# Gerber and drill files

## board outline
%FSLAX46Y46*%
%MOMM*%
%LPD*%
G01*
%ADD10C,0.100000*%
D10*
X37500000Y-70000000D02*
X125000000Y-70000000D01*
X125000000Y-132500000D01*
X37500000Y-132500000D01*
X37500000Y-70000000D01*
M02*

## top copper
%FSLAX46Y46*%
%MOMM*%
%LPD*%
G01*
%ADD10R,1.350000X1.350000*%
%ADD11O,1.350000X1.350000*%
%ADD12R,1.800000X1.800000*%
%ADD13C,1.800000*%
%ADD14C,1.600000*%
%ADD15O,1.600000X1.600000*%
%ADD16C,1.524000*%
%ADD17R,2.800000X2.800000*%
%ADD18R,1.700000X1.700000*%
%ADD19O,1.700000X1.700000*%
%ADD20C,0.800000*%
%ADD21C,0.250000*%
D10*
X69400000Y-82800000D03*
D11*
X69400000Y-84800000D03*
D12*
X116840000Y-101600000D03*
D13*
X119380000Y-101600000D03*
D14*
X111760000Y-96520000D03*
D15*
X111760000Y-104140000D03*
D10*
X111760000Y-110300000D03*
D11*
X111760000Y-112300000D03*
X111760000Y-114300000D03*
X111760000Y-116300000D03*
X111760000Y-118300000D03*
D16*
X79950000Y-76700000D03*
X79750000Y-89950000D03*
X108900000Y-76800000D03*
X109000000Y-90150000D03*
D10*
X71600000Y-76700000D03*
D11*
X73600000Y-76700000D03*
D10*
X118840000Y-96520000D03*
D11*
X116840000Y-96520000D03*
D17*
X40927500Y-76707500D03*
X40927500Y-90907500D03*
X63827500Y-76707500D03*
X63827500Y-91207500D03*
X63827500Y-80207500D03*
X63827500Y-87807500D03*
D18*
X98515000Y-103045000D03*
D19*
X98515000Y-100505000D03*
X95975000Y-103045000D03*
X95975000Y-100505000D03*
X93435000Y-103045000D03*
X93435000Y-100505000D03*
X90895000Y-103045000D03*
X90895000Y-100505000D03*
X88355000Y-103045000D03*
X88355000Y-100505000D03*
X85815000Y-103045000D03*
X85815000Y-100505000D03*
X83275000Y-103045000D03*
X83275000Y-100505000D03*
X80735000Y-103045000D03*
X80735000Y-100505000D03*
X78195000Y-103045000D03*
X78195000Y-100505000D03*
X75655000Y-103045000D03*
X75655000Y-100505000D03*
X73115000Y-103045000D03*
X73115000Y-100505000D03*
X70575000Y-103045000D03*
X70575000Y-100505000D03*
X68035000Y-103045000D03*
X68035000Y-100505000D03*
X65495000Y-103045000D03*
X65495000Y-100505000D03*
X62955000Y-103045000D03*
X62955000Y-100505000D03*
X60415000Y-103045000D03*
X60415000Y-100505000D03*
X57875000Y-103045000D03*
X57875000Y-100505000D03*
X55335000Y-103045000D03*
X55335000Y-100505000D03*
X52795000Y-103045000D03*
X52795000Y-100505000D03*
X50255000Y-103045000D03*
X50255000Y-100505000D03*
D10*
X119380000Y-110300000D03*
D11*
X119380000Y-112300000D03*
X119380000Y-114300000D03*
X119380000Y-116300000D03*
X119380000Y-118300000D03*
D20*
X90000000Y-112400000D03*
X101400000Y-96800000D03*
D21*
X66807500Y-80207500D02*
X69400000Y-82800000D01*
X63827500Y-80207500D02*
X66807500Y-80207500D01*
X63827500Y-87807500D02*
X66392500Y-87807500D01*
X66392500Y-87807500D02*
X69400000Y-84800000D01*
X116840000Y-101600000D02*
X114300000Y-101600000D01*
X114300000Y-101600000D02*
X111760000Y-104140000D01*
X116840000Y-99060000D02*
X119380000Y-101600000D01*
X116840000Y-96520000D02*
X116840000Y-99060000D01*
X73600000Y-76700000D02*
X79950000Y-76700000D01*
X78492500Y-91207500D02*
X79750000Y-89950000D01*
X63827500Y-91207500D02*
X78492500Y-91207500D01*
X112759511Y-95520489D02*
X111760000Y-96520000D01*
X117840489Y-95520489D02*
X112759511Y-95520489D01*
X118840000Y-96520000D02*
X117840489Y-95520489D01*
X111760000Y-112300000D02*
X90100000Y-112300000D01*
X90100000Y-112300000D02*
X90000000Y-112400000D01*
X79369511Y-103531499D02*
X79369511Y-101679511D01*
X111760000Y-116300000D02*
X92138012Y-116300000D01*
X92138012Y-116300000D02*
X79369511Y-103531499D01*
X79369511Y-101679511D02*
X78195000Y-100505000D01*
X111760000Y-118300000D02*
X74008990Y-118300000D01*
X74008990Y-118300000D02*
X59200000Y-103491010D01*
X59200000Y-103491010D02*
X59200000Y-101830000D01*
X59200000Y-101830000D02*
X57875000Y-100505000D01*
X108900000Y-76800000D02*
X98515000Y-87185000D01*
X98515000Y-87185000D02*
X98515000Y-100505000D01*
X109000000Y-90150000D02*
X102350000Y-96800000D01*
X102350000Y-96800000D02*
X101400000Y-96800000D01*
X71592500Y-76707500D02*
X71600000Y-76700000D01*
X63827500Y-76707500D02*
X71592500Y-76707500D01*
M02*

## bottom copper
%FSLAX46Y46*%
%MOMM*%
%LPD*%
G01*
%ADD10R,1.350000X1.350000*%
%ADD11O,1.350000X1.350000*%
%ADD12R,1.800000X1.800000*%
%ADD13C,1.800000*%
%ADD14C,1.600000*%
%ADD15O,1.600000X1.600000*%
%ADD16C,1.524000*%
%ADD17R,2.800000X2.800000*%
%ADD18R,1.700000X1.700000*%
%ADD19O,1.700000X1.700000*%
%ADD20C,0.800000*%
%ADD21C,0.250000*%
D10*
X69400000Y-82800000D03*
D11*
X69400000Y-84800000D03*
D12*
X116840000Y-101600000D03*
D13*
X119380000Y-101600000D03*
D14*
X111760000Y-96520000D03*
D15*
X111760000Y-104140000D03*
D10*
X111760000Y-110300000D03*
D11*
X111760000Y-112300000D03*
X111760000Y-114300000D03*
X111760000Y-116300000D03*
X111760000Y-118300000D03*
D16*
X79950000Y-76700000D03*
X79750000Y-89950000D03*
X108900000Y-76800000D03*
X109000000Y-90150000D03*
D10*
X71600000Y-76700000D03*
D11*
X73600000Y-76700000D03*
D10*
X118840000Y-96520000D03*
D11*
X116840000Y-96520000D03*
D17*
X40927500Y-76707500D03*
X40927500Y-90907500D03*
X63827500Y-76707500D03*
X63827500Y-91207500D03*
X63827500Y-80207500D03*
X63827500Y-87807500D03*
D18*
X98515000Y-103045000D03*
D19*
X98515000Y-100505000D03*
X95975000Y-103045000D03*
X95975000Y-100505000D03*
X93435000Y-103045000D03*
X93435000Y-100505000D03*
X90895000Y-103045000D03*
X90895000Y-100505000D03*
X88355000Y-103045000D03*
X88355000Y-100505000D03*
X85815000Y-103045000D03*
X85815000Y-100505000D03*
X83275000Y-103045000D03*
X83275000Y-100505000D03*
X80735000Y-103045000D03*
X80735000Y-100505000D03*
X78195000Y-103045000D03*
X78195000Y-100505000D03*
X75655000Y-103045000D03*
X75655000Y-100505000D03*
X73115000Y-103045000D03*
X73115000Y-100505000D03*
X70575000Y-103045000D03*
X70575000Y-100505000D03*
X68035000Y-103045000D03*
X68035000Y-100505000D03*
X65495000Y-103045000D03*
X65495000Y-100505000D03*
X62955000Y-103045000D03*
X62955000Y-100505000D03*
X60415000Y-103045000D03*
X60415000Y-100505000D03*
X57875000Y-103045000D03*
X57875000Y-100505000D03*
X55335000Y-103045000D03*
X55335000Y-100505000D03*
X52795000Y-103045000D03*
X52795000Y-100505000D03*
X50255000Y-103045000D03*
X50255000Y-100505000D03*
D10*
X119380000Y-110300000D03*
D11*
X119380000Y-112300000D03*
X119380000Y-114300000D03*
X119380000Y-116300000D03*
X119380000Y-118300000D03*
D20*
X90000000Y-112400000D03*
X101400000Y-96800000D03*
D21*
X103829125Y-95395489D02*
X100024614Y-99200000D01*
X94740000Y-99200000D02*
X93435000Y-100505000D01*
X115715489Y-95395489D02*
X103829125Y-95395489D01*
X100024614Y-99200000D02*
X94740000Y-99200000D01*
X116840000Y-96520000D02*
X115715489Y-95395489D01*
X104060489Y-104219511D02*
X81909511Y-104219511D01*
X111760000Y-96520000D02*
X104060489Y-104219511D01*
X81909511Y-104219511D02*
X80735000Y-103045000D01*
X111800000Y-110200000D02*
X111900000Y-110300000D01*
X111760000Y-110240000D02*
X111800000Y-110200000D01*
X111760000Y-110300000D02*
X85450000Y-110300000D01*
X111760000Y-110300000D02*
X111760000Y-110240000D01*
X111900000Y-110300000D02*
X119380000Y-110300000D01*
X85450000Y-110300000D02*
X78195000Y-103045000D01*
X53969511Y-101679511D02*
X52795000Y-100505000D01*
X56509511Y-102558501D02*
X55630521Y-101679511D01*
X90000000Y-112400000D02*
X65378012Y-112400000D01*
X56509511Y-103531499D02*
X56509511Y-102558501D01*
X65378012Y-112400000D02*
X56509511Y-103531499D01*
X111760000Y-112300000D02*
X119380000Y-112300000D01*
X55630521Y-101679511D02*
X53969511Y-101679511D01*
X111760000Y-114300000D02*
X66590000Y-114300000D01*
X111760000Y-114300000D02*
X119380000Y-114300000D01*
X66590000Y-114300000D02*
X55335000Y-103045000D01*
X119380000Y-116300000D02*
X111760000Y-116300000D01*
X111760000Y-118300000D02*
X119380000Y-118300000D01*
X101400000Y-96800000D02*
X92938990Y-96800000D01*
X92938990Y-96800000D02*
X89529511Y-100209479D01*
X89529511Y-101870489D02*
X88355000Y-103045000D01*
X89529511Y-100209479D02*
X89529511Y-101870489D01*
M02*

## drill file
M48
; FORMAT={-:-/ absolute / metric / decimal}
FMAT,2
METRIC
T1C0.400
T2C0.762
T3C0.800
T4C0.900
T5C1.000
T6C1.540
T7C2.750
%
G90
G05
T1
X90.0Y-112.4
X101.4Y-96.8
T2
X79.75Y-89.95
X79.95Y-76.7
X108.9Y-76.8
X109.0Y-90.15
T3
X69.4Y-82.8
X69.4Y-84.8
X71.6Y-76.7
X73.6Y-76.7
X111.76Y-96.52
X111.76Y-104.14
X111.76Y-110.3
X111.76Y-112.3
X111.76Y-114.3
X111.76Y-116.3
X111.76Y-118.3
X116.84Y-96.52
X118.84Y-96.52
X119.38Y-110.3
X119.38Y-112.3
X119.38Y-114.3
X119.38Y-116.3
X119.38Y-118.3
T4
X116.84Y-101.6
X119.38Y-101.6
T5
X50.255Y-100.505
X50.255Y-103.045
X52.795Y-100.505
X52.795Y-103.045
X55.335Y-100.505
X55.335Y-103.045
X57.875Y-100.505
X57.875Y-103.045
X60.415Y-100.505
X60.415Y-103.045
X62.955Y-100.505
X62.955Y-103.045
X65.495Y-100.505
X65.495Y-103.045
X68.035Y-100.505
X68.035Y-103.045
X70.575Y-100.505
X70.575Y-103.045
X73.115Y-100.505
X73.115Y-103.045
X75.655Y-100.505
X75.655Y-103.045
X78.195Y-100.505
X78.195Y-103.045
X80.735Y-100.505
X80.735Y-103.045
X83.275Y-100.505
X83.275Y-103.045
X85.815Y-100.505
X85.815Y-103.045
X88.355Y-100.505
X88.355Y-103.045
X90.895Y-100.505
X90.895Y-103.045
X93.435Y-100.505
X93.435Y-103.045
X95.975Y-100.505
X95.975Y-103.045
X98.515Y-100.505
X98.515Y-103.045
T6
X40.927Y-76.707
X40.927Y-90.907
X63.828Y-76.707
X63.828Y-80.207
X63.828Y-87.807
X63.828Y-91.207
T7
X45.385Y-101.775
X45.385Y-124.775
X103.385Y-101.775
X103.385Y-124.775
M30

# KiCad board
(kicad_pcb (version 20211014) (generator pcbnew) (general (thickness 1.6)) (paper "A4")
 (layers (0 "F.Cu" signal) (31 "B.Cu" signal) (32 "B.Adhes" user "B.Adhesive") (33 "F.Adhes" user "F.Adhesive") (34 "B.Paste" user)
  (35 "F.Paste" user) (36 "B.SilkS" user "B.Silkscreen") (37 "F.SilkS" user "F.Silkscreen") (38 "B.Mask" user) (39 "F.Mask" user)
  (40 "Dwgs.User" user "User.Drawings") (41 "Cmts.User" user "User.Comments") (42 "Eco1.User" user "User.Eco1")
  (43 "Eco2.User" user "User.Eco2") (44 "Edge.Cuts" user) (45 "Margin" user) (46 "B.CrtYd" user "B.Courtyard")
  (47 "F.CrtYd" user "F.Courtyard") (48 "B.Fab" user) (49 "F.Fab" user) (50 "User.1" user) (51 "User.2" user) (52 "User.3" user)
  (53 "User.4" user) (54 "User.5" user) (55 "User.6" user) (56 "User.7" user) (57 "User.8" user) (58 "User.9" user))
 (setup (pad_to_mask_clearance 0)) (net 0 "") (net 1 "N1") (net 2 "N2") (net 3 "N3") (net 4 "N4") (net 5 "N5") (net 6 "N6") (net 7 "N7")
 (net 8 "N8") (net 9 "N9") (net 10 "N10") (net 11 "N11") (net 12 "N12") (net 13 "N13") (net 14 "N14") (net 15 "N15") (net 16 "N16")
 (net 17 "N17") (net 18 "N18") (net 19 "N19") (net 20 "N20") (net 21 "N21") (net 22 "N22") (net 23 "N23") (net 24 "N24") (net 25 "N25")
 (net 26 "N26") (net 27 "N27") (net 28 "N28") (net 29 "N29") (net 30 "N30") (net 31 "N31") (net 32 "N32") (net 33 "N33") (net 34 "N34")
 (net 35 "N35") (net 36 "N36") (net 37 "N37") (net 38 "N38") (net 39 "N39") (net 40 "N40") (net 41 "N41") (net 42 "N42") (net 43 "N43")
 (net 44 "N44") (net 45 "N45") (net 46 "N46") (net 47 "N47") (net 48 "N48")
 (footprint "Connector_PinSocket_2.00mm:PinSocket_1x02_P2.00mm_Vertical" (layer "F.Cu") (at 69.4 82.8)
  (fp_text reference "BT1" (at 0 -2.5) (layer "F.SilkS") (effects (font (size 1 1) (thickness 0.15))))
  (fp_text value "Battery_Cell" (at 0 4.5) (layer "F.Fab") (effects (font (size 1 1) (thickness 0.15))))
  (pad "1" thru_hole rect (at 0 0) (size 1.35 1.35) (drill 0.8) (layers *.Cu *.Mask) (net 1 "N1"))
  (pad "2" thru_hole oval (at 0 2) (size 1.35 1.35) (drill 0.8) (layers *.Cu *.Mask) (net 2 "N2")))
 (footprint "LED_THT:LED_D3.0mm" (layer "F.Cu") (at 116.84 101.6)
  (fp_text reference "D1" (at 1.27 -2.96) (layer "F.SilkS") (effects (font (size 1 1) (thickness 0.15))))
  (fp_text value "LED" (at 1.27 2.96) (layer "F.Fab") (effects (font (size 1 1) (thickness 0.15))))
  (pad "1" thru_hole rect (at 0 0) (size 1.8 1.8) (drill 0.9) (layers *.Cu *.Mask) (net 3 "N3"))
  (pad "2" thru_hole circle (at 2.54 0) (size 1.8 1.8) (drill 0.9) (layers *.Cu *.Mask) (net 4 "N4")))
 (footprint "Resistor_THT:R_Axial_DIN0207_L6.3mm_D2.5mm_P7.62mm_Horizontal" (layer "F.Cu") (at 111.76 96.52 -90)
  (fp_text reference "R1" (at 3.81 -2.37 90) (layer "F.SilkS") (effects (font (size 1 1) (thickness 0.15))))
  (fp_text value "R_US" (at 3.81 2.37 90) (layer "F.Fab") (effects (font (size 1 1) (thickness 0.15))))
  (pad "1" thru_hole circle (at 0 0 270) (size 1.6 1.6) (drill 0.8) (layers *.Cu *.Mask) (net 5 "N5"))
  (pad "2" thru_hole oval (at 7.62 0 270) (size 1.6 1.6) (drill 0.8) (layers *.Cu *.Mask) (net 3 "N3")))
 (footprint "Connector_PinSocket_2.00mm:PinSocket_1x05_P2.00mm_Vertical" (layer "F.Cu") (at 111.76 110.3)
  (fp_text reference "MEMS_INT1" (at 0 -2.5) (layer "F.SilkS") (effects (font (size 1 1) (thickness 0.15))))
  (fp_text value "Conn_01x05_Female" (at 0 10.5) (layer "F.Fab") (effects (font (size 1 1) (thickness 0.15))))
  (pad "1" thru_hole rect (at 0 0) (size 1.35 1.35) (drill 0.8) (layers *.Cu *.Mask) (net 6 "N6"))
  (pad "2" thru_hole oval (at 0 2) (size 1.35 1.35) (drill 0.8) (layers *.Cu *.Mask) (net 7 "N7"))
  (pad "3" thru_hole oval (at 0 4) (size 1.35 1.35) (drill 0.8) (layers *.Cu *.Mask) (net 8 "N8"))
  (pad "4" thru_hole oval (at 0 6) (size 1.35 1.35) (drill 0.8) (layers *.Cu *.Mask) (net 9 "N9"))
  (pad "5" thru_hole oval (at 0 8) (size 1.35 1.35) (drill 0.8) (layers *.Cu *.Mask) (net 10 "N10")))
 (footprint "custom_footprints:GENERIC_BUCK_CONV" (layer "F.Cu") (at 94.2 83.6)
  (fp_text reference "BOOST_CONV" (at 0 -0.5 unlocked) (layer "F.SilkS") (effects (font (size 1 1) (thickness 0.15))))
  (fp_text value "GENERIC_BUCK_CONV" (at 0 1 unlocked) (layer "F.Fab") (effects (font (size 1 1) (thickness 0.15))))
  (pad "1" thru_hole circle (at -14.25 -6.9) (size 1.524 1.524) (drill 0.762) (layers *.Cu *.Mask) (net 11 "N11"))
  (pad "2" thru_hole circle (at -14.45 6.35) (size 1.524 1.524) (drill 0.762) (layers *.Cu *.Mask) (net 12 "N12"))
  (pad "3" thru_hole circle (at 14.7 -6.8) (size 1.524 1.524) (drill 0.762) (layers *.Cu *.Mask) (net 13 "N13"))
  (pad "4" thru_hole circle (at 14.8 6.55) (size 1.524 1.524) (drill 0.762) (layers *.Cu *.Mask) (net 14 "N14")))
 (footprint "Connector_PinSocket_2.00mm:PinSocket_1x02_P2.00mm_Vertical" (layer "F.Cu") (at 71.6 76.7 90)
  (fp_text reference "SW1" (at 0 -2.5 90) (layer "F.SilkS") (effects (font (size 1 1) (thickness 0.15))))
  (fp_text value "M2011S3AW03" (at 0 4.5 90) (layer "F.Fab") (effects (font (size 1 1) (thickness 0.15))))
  (pad "1" thru_hole rect (at 0 0 90) (size 1.35 1.35) (drill 0.8) (layers *.Cu *.Mask) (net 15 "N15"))
  (pad "2" thru_hole oval (at 0 2 90) (size 1.35 1.35) (drill 0.8) (layers *.Cu *.Mask) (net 11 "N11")))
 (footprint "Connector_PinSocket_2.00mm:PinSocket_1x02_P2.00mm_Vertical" (layer "F.Cu") (at 118.84 96.52 -90)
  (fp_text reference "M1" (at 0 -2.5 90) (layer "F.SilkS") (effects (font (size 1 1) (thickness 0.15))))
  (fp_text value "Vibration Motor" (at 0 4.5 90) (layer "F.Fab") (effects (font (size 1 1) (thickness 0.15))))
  (pad "1" thru_hole rect (at 0 0 270) (size 1.35 1.35) (drill 0.8) (layers *.Cu *.Mask) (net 5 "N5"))
  (pad "2" thru_hole oval (at 0 2 270) (size 1.35 1.35) (drill 0.8) (layers *.Cu *.Mask) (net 4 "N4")))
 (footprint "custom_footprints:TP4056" (layer "F.Cu") (at 39.2275 75.0075)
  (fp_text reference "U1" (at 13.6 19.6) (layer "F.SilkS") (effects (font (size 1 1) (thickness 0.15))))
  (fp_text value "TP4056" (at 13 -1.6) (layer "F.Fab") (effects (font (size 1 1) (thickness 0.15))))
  (pad "1" thru_hole rect (at 1.7 1.7) (size 2.8 2.8) (drill 1.54) (layers *.Cu *.Mask) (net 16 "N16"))
  (pad "2" thru_hole rect (at 1.7 15.9) (size 2.8 2.8) (drill 1.54) (layers *.Cu *.Mask) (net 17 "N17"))
  (pad "3" thru_hole rect (at 24.6 1.7) (size 2.8 2.8) (drill 1.54) (layers *.Cu *.Mask) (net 15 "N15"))
  (pad "4" thru_hole rect (at 24.6 16.2) (size 2.8 2.8) (drill 1.54) (layers *.Cu *.Mask) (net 12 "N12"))
  (pad "5" thru_hole rect (at 24.6 5.2) (size 2.8 2.8) (drill 1.54) (layers *.Cu *.Mask) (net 1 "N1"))
  (pad "6" thru_hole rect (at 24.6 12.8) (size 2.8 2.8) (drill 1.54) (layers *.Cu *.Mask) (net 2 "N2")))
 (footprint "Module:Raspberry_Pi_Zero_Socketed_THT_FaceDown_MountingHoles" (layer "F.Cu") (at 98.515 103.045 -90)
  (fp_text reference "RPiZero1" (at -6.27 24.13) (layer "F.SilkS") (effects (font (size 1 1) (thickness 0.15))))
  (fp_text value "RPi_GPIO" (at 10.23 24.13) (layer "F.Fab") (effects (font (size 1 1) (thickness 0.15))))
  (pad "" np_thru_hole circle (at 21.73 -4.87) (size 2.75 2.75) (drill 2.75) (layers *.Cu *.Mask) (solder_mask_margin 1.625))
  (pad "" np_thru_hole circle (at -1.27 53.13) (size 2.75 2.75) (drill 2.75) (layers *.Cu *.Mask) (solder_mask_margin 1.625))
  (pad "" np_thru_hole circle (at -1.27 -4.87) (size 2.75 2.75) (drill 2.75) (layers *.Cu *.Mask) (solder_mask_margin 1.625))
  (pad "" np_thru_hole circle (at 21.73 53.13) (size 2.75 2.75) (drill 2.75) (layers *.Cu *.Mask) (solder_mask_margin 1.625))
  (pad "1" thru_hole rect (at 0 0 270) (size 1.7 1.7) (drill 1) (layers *.Cu *.Mask) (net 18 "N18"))
  (pad "2" thru_hole oval (at -2.54 0 270) (size 1.7 1.7) (drill 1) (layers *.Cu *.Mask) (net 13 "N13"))
  (pad "3" thru_hole oval (at 0 2.54 270) (size 1.7 1.7) (drill 1) (layers *.Cu *.Mask) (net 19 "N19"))
  (pad "4" thru_hole oval (at -2.54 2.54 270) (size 1.7 1.7) (drill 1) (layers *.Cu *.Mask) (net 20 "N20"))
  (pad "5" thru_hole oval (at 0 5.08 270) (size 1.7 1.7) (drill 1) (layers *.Cu *.Mask) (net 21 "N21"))
  (pad "6" thru_hole oval (at -2.54 5.08 270) (size 1.7 1.7) (drill 1) (layers *.Cu *.Mask) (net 4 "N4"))
  (pad "7" thru_hole oval (at 0 7.62 270) (size 1.7 1.7) (drill 1) (layers *.Cu *.Mask) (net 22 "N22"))
  (pad "8" thru_hole oval (at -2.54 7.62 270) (size 1.7 1.7) (drill 1) (layers *.Cu *.Mask) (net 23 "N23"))
  (pad "9" thru_hole oval (at 0 10.16 270) (size 1.7 1.7) (drill 1) (layers *.Cu *.Mask) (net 14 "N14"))
  (pad "10" thru_hole oval (at -2.54 10.16 270) (size 1.7 1.7) (drill 1) (layers *.Cu *.Mask) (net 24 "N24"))
  (pad "11" thru_hole oval (at 0 12.7 270) (size 1.7 1.7) (drill 1) (layers *.Cu *.Mask) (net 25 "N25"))
  (pad "12" thru_hole oval (at -2.54 12.7 270) (size 1.7 1.7) (drill 1) (layers *.Cu *.Mask) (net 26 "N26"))
  (pad "13" thru_hole oval (at 0 15.24 270) (size 1.7 1.7) (drill 1) (layers *.Cu *.Mask) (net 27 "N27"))
  (pad "14" thru_hole oval (at -2.54 15.24 270) (size 1.7 1.7) (drill 1) (layers *.Cu *.Mask) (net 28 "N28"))
  (pad "15" thru_hole oval (at 0 17.78 270) (size 1.7 1.7) (drill 1) (layers *.Cu *.Mask) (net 5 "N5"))
  (pad "16" thru_hole oval (at -2.54 17.78 270) (size 1.7 1.7) (drill 1) (layers *.Cu *.Mask) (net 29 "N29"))
  (pad "17" thru_hole oval (at 0 20.32 270) (size 1.7 1.7) (drill 1) (layers *.Cu *.Mask) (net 6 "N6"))
  (pad "18" thru_hole oval (at -2.54 20.32 270) (size 1.7 1.7) (drill 1) (layers *.Cu *.Mask) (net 9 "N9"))
  (pad "19" thru_hole oval (at 0 22.86 270) (size 1.7 1.7) (drill 1) (layers *.Cu *.Mask) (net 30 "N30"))
  (pad "20" thru_hole oval (at -2.54 22.86 270) (size 1.7 1.7) (drill 1) (layers *.Cu *.Mask) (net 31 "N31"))
  (pad "21" thru_hole oval (at 0 25.4 270) (size 1.7 1.7) (drill 1) (layers *.Cu *.Mask) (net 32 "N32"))
  (pad "22" thru_hole oval (at -2.54 25.4 270) (size 1.7 1.7) (drill 1) (layers *.Cu *.Mask) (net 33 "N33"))
  (pad "23" thru_hole oval (at 0 27.94 270) (size 1.7 1.7) (drill 1) (layers *.Cu *.Mask) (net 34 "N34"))
  (pad "24" thru_hole oval (at -2.54 27.94 270) (size 1.7 1.7) (drill 1) (layers *.Cu *.Mask) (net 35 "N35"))
  (pad "25" thru_hole oval (at 0 30.48 270) (size 1.7 1.7) (drill 1) (layers *.Cu *.Mask) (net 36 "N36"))
  (pad "26" thru_hole oval (at -2.54 30.48 270) (size 1.7 1.7) (drill 1) (layers *.Cu *.Mask) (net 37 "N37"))
  (pad "27" thru_hole oval (at 0 33.02 270) (size 1.7 1.7) (drill 1) (layers *.Cu *.Mask) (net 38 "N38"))
  (pad "28" thru_hole oval (at -2.54 33.02 270) (size 1.7 1.7) (drill 1) (layers *.Cu *.Mask) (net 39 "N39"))
  (pad "29" thru_hole oval (at 0 35.56 270) (size 1.7 1.7) (drill 1) (layers *.Cu *.Mask) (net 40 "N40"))
  (pad "30" thru_hole oval (at -2.54 35.56 270) (size 1.7 1.7) (drill 1) (layers *.Cu *.Mask) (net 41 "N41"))
  (pad "31" thru_hole oval (at 0 38.1 270) (size 1.7 1.7) (drill 1) (layers *.Cu *.Mask) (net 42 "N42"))
  (pad "32" thru_hole oval (at -2.54 38.1 270) (size 1.7 1.7) (drill 1) (layers *.Cu *.Mask) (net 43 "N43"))
  (pad "33" thru_hole oval (at 0 40.64 270) (size 1.7 1.7) (drill 1) (layers *.Cu *.Mask) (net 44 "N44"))
  (pad "34" thru_hole oval (at -2.54 40.64 270) (size 1.7 1.7) (drill 1) (layers *.Cu *.Mask) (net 10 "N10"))
  (pad "35" thru_hole oval (at 0 43.18 270) (size 1.7 1.7) (drill 1) (layers *.Cu *.Mask) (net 8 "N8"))
  (pad "36" thru_hole oval (at -2.54 43.18 270) (size 1.7 1.7) (drill 1) (layers *.Cu *.Mask) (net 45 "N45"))
  (pad "37" thru_hole oval (at 0 45.72 270) (size 1.7 1.7) (drill 1) (layers *.Cu *.Mask) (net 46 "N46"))
  (pad "38" thru_hole oval (at -2.54 45.72 270) (size 1.7 1.7) (drill 1) (layers *.Cu *.Mask) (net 7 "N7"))
  (pad "39" thru_hole oval (at 0 48.26 270) (size 1.7 1.7) (drill 1) (layers *.Cu *.Mask) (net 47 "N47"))
  (pad "40" thru_hole oval (at -2.54 48.26 270) (size 1.7 1.7) (drill 1) (layers *.Cu *.Mask) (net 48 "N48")))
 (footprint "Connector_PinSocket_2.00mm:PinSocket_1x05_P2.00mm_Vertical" (layer "F.Cu") (at 119.38 110.3)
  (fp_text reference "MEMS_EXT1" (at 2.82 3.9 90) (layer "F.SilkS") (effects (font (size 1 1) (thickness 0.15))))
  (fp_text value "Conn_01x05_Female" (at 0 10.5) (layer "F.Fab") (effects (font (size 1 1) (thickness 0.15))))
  (pad "1" thru_hole rect (at 0 0) (size 1.35 1.35) (drill 0.8) (layers *.Cu *.Mask) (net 6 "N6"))
  (pad "2" thru_hole oval (at 0 2) (size 1.35 1.35) (drill 0.8) (layers *.Cu *.Mask) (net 7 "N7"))
  (pad "3" thru_hole oval (at 0 4) (size 1.35 1.35) (drill 0.8) (layers *.Cu *.Mask) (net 8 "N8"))
  (pad "4" thru_hole oval (at 0 6) (size 1.35 1.35) (drill 0.8) (layers *.Cu *.Mask) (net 9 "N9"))
  (pad "5" thru_hole oval (at 0 8) (size 1.35 1.35) (drill 0.8) (layers *.Cu *.Mask) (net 10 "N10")))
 (gr_rect (start 37.5 70) (end 125 132.5) (layer "Edge.Cuts") (width 0.1) (fill none))
 (segment (start 66.8075 80.2075) (end 69.4 82.8) (width 0.25) (layer "F.Cu") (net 1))
 (segment (start 63.8275 80.2075) (end 66.8075 80.2075) (width 0.25) (layer "F.Cu") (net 1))
 (segment (start 63.8275 87.8075) (end 66.3925 87.8075) (width 0.25) (layer "F.Cu") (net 2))
 (segment (start 66.3925 87.8075) (end 69.4 84.8) (width 0.25) (layer "F.Cu") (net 2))
 (segment (start 116.84 101.6) (end 114.3 101.6) (width 0.25) (layer "F.Cu") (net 3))
 (segment (start 114.3 101.6) (end 111.76 104.14) (width 0.25) (layer "F.Cu") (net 3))
 (segment (start 116.84 99.06) (end 119.38 101.6) (width 0.25) (layer "F.Cu") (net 4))
 (segment (start 116.84 96.52) (end 116.84 99.06) (width 0.25) (layer "F.Cu") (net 4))
 (segment (start 103.829125 95.395489) (end 100.024614 99.2) (width 0.25) (layer "B.Cu") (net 4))
 (segment (start 94.74 99.2) (end 93.435 100.505) (width 0.25) (layer "B.Cu") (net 4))
 (segment (start 115.715489 95.395489) (end 103.829125 95.395489) (width 0.25) (layer "B.Cu") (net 4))
 (segment (start 100.024614 99.2) (end 94.74 99.2) (width 0.25) (layer "B.Cu") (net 4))
 (segment (start 116.84 96.52) (end 115.715489 95.395489) (width 0.25) (layer "B.Cu") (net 4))
 (segment (start 73.6 76.7) (end 79.95 76.7) (width 0.25) (layer "F.Cu") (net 11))
 (segment (start 78.4925 91.2075) (end 79.75 89.95) (width 0.25) (layer "F.Cu") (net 12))
 (segment (start 63.8275 91.2075) (end 78.4925 91.2075) (width 0.25) (layer "F.Cu") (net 12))
 (segment (start 112.759511 95.520489) (end 111.76 96.52) (width 0.25) (layer "F.Cu") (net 5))
 (segment (start 117.840489 95.520489) (end 112.759511 95.520489) (width 0.25) (layer "F.Cu") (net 5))
 (segment (start 118.84 96.52) (end 117.840489 95.520489) (width 0.25) (layer "F.Cu") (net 5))
 (segment (start 104.060489 104.219511) (end 81.909511 104.219511) (width 0.25) (layer "B.Cu") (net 5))
 (segment (start 111.76 96.52) (end 104.060489 104.219511) (width 0.25) (layer "B.Cu") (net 5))
 (segment (start 81.909511 104.219511) (end 80.735 103.045) (width 0.25) (layer "B.Cu") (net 5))
 (segment (start 111.8 110.2) (end 111.9 110.3) (width 0.25) (layer "B.Cu") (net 6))
 (segment (start 111.76 110.24) (end 111.8 110.2) (width 0.25) (layer "B.Cu") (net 6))
 (segment (start 111.76 110.3) (end 85.45 110.3) (width 0.25) (layer "B.Cu") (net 6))
 (segment (start 111.76 110.3) (end 111.76 110.24) (width 0.25) (layer "B.Cu") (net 6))
 (segment (start 111.9 110.3) (end 119.38 110.3) (width 0.25) (layer "B.Cu") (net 6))
 (segment (start 85.45 110.3) (end 78.195 103.045) (width 0.25) (layer "B.Cu") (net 6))
 (segment (start 111.76 112.3) (end 90.1 112.3) (width 0.25) (layer "F.Cu") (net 7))
 (segment (start 90.1 112.3) (end 90 112.4) (width 0.25) (layer "F.Cu") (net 7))
 (via (at 90 112.4) (size 0.8) (drill 0.4) (layers "F.Cu" "B.Cu") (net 7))
 (segment (start 53.969511 101.679511) (end 52.795 100.505) (width 0.25) (layer "B.Cu") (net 7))
 (segment (start 56.509511 102.558501) (end 55.630521 101.679511) (width 0.25) (layer "B.Cu") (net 7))
 (segment (start 90 112.4) (end 65.378012 112.4) (width 0.25) (layer "B.Cu") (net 7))
 (segment (start 56.509511 103.531499) (end 56.509511 102.558501) (width 0.25) (layer "B.Cu") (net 7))
 (segment (start 65.378012 112.4) (end 56.509511 103.531499) (width 0.25) (layer "B.Cu") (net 7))
 (segment (start 111.76 112.3) (end 119.38 112.3) (width 0.25) (layer "B.Cu") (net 7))
 (segment (start 55.630521 101.679511) (end 53.969511 101.679511) (width 0.25) (layer "B.Cu") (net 7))
 (segment (start 111.76 114.3) (end 66.59 114.3) (width 0.25) (layer "B.Cu") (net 8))
 (segment (start 111.76 114.3) (end 119.38 114.3) (width 0.25) (layer "B.Cu") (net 8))
 (segment (start 66.59 114.3) (end 55.335 103.045) (width 0.25) (layer "B.Cu") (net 8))
 (segment (start 79.369511 103.531499) (end 79.369511 101.679511) (width 0.25) (layer "F.Cu") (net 9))
 (segment (start 111.76 116.3) (end 92.138012 116.3) (width 0.25) (layer "F.Cu") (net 9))
 (segment (start 92.138012 116.3) (end 79.369511 103.531499) (width 0.25) (layer "F.Cu") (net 9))
 (segment (start 79.369511 101.679511) (end 78.195 100.505) (width 0.25) (layer "F.Cu") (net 9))
 (segment (start 119.38 116.3) (end 111.76 116.3) (width 0.25) (layer "B.Cu") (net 9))
 (segment (start 111.76 118.3) (end 74.00899 118.3) (width 0.25) (layer "F.Cu") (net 10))
 (segment (start 74.00899 118.3) (end 59.2 103.49101) (width 0.25) (layer "F.Cu") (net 10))
 (segment (start 59.2 103.49101) (end 59.2 101.83) (width 0.25) (layer "F.Cu") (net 10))
 (segment (start 59.2 101.83) (end 57.875 100.505) (width 0.25) (layer "F.Cu") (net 10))
 (segment (start 111.76 118.3) (end 119.38 118.3) (width 0.25) (layer "B.Cu") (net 10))
 (segment (start 108.9 76.8) (end 98.515 87.185) (width 0.25) (layer "F.Cu") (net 13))
 (segment (start 98.515 87.185) (end 98.515 100.505) (width 0.25) (layer "F.Cu") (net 13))
 (segment (start 109 90.15) (end 102.35 96.8) (width 0.25) (layer "F.Cu") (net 14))
 (segment (start 102.35 96.8) (end 101.4 96.8) (width 0.25) (layer "F.Cu") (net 14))
 (via (at 101.4 96.8) (size 0.8) (drill 0.4) (layers "F.Cu" "B.Cu") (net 14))
 (segment (start 101.4 96.8) (end 92.93899 96.8) (width 0.25) (layer "B.Cu") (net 14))
 (segment (start 92.93899 96.8) (end 89.529511 100.209479) (width 0.25) (layer "B.Cu") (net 14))
 (segment (start 89.529511 101.870489) (end 88.355 103.045) (width 0.25) (layer "B.Cu") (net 14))
 (segment (start 89.529511 100.209479) (end 89.529511 101.870489) (width 0.25) (layer "B.Cu") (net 14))
 (segment (start 71.5925 76.7075) (end 71.6 76.7) (width 0.25) (layer "F.Cu") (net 15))
 (segment (start 63.8275 76.7075) (end 71.5925 76.7075) (width 0.25) (layer "F.Cu") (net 15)))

